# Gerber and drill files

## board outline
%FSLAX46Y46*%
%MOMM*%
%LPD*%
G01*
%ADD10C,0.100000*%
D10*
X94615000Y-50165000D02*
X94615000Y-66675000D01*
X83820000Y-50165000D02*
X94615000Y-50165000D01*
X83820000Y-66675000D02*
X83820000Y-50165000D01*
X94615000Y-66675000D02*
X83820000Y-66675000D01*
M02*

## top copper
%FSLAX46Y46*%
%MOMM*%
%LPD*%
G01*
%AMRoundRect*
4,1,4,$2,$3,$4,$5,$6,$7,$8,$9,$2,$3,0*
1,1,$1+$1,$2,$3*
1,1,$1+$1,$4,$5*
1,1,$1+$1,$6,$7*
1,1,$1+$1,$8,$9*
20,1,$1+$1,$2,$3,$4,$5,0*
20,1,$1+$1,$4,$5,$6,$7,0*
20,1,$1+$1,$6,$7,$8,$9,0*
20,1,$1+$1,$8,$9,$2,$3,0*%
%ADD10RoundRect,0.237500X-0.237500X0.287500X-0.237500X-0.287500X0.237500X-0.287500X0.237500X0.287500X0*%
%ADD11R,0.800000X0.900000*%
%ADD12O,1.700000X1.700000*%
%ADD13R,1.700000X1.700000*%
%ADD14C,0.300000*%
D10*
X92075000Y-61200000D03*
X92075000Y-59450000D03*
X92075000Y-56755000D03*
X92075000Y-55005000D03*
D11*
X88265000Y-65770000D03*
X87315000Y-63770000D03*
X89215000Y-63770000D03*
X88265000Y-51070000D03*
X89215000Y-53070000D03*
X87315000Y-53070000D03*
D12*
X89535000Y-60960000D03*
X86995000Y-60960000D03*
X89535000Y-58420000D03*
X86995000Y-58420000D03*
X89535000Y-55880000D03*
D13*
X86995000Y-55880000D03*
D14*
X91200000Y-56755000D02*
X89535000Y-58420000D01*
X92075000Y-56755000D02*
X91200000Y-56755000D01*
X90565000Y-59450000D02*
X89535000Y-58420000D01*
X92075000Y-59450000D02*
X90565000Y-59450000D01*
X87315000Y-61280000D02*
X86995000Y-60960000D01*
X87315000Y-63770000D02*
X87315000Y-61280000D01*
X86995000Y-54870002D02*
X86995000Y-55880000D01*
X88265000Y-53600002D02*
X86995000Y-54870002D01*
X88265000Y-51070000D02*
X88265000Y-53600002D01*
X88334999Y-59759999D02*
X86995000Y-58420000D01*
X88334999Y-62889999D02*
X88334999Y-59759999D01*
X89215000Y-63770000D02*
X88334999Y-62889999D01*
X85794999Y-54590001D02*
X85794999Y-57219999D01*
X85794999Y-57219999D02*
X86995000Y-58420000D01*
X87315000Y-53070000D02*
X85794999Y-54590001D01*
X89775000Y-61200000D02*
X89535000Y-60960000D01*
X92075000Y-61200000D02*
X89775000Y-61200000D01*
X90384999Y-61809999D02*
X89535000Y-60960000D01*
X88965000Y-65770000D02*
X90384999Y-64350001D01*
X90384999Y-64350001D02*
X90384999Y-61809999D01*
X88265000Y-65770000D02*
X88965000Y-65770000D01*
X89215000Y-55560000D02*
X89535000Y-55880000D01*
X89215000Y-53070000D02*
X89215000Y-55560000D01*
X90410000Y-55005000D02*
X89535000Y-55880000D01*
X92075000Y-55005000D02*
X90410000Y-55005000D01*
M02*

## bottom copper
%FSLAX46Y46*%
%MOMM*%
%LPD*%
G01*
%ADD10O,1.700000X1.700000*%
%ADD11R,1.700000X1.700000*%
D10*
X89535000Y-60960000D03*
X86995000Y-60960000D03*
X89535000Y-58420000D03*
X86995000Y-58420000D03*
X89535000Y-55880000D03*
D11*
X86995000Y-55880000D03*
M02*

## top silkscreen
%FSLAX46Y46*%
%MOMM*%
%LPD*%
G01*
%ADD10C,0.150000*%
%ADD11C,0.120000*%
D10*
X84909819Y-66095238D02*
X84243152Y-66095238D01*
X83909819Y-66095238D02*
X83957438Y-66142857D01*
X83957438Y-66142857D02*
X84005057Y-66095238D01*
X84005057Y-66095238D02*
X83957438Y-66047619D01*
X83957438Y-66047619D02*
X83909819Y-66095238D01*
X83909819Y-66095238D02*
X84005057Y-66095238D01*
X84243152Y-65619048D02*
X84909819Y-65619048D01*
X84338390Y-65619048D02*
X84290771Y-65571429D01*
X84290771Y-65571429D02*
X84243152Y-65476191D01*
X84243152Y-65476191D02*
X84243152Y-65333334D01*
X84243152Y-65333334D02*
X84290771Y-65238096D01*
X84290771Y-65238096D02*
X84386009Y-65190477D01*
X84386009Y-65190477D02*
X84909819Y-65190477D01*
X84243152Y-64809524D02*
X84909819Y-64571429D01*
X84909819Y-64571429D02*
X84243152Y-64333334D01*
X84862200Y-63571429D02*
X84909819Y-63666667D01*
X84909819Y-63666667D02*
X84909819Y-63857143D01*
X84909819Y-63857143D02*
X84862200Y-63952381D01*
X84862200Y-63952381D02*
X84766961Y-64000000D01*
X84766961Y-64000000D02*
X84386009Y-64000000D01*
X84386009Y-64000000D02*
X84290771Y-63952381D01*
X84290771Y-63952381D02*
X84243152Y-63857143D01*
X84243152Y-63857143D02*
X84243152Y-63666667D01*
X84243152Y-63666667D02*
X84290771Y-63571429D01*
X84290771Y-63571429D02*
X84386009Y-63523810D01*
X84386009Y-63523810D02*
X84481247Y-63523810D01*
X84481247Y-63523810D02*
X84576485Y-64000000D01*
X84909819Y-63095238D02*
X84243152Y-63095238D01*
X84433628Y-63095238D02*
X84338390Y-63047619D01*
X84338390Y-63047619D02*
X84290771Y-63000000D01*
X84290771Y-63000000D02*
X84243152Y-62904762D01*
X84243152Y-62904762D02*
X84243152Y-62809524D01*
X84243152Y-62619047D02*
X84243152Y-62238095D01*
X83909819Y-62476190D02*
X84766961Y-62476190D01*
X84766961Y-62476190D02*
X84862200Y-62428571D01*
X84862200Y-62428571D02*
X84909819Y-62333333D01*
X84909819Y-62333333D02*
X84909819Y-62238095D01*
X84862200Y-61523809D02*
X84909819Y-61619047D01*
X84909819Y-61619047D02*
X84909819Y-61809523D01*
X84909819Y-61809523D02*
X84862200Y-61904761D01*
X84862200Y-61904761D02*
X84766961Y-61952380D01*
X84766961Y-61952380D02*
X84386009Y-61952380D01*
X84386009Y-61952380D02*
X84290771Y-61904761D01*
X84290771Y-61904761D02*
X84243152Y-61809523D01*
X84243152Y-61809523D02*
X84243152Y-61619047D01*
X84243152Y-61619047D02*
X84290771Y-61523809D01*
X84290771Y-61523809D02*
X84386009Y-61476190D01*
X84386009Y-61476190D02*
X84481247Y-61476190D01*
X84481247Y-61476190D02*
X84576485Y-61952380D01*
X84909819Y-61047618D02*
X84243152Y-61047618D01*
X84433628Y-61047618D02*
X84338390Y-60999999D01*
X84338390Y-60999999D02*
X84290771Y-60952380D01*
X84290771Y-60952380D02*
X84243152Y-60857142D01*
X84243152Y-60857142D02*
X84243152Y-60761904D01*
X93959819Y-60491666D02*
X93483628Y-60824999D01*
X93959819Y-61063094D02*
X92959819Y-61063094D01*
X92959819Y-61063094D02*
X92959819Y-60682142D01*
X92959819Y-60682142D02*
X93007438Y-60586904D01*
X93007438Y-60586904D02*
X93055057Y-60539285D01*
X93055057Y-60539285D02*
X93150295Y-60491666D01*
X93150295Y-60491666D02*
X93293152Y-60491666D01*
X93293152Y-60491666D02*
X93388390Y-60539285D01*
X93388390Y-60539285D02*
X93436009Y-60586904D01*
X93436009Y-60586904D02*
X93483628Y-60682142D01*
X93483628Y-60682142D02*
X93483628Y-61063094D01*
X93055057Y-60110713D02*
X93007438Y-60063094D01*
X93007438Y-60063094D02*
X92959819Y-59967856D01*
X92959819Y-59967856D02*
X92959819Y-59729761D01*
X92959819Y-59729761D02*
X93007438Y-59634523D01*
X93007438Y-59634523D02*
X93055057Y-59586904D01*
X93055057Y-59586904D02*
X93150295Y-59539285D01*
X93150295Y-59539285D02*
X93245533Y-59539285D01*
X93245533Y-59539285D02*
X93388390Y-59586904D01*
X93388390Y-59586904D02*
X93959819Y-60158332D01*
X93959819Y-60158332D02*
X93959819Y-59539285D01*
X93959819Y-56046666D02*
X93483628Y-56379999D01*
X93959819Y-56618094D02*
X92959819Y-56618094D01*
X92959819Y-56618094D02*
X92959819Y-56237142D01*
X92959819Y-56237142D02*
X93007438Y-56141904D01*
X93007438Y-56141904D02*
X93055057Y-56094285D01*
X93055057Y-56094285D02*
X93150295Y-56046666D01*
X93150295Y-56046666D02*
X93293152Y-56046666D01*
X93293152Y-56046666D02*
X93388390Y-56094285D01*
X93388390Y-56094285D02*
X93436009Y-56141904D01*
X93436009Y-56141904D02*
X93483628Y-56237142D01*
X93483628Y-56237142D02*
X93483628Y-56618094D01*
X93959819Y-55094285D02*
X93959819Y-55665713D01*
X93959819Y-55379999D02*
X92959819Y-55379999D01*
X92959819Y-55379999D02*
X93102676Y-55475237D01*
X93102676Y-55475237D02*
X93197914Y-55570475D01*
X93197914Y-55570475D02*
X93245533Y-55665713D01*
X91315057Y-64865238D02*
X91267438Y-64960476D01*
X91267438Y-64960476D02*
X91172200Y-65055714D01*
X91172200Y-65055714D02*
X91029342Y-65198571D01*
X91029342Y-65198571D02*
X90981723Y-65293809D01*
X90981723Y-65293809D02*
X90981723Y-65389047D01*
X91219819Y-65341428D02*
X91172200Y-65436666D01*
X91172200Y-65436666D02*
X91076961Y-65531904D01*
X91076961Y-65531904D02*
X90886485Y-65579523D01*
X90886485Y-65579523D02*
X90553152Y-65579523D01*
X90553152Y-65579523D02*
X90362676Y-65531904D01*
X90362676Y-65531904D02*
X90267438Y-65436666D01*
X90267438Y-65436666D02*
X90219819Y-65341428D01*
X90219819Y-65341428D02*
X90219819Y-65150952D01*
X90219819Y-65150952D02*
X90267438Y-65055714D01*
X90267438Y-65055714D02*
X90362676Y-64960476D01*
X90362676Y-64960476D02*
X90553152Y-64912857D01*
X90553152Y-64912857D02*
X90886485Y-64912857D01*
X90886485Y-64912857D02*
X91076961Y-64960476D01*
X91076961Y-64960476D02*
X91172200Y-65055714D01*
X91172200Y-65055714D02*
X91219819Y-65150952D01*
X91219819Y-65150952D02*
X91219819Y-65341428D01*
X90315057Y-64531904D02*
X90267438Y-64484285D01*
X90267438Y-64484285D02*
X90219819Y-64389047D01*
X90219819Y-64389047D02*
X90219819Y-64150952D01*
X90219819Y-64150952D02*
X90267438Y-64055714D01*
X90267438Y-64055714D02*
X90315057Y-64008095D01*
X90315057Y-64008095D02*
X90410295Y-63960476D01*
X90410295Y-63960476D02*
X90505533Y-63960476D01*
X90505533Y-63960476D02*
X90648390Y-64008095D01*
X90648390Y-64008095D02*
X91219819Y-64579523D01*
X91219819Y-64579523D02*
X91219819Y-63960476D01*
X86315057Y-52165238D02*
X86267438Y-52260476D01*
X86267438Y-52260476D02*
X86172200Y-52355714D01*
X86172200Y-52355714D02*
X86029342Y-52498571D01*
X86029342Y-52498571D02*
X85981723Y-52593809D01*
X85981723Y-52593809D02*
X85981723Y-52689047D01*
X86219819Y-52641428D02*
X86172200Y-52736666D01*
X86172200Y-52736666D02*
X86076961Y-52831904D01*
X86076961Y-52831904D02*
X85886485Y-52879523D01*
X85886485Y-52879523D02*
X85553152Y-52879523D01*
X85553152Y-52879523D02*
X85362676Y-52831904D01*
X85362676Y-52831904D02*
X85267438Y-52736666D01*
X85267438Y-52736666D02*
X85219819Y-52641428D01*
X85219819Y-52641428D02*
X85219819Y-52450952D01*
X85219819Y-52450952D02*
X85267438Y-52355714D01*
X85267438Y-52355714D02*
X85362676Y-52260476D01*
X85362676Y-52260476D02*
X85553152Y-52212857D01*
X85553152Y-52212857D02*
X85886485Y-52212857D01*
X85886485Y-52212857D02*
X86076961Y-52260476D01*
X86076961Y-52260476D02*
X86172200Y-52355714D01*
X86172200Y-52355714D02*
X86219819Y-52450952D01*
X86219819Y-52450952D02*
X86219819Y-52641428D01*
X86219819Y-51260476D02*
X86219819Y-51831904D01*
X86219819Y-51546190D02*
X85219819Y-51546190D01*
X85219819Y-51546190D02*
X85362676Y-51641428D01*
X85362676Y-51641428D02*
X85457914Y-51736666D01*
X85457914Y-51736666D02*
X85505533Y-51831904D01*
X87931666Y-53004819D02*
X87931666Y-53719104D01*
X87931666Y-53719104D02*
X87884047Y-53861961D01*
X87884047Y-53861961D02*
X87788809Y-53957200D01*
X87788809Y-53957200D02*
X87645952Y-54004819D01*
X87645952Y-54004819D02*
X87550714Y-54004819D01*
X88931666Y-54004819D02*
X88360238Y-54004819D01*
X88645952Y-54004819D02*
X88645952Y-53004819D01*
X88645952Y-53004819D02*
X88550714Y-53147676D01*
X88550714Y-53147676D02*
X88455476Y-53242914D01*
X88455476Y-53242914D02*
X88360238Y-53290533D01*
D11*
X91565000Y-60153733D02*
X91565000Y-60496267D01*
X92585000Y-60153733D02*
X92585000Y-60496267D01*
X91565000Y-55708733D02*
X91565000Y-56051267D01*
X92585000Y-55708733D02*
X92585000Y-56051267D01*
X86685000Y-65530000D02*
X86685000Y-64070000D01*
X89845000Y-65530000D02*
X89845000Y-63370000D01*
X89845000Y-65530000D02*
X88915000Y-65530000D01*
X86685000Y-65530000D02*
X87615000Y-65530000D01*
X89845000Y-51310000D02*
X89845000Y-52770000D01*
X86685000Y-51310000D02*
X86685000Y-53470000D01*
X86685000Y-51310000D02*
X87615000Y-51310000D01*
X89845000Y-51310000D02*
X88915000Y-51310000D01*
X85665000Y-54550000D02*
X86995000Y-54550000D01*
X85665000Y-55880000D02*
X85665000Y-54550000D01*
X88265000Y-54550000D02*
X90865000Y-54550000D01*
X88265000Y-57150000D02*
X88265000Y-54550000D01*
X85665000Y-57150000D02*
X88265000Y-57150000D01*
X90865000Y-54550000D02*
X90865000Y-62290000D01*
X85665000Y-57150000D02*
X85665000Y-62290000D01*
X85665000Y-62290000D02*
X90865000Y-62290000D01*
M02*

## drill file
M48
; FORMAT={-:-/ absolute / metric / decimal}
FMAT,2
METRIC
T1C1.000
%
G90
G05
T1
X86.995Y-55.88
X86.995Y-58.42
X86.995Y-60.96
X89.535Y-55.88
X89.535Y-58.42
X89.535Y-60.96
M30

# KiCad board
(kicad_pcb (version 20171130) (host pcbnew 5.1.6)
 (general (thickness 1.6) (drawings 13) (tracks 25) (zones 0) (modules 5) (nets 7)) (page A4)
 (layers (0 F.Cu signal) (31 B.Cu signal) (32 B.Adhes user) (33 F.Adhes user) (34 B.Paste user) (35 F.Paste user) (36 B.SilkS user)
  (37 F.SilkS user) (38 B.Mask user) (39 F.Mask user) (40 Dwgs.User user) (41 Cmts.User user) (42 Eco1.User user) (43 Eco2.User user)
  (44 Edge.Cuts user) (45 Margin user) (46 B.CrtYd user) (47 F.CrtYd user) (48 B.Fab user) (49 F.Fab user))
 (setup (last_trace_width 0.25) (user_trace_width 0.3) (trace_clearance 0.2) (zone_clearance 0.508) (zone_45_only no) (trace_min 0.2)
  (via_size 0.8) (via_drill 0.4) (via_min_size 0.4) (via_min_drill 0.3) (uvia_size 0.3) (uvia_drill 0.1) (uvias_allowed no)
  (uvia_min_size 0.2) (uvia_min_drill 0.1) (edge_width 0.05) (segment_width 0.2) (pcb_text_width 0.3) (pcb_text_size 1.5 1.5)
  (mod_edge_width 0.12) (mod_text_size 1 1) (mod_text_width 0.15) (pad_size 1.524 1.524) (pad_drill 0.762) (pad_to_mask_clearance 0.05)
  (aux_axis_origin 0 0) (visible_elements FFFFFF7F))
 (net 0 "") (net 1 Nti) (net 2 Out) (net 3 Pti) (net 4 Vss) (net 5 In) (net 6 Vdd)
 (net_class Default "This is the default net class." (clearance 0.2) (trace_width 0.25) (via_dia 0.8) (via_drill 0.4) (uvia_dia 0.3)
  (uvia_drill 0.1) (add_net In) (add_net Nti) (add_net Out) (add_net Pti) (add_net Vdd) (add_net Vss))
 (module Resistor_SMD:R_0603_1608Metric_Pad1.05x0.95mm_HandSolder (layer F.Cu) (at 92.075 60.325 270)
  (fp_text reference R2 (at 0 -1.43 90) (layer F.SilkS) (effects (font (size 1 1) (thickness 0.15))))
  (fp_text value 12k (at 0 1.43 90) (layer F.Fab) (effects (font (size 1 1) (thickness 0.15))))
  (fp_line (start -0.171267 0.51) (end 0.171267 0.51) (layer F.SilkS) (width 0.12))
  (fp_line (start -0.171267 -0.51) (end 0.171267 -0.51) (layer F.SilkS) (width 0.12))
  (pad 2 smd roundrect (at 0.875 0 270) (size 1.05 0.95) (layers F.Cu F.Paste F.Mask) (roundrect_rratio 0.25) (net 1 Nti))
  (pad 1 smd roundrect (at -0.875 0 270) (size 1.05 0.95) (layers F.Cu F.Paste F.Mask) (roundrect_rratio 0.25) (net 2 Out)))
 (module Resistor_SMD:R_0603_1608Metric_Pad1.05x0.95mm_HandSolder (layer F.Cu) (at 92.075 55.88 270)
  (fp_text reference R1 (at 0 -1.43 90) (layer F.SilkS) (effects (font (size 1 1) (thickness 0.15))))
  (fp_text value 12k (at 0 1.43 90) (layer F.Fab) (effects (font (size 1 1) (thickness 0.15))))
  (fp_line (start -0.171267 0.51) (end 0.171267 0.51) (layer F.SilkS) (width 0.12))
  (fp_line (start -0.171267 -0.51) (end 0.171267 -0.51) (layer F.SilkS) (width 0.12))
  (pad 2 smd roundrect (at 0.875 0 270) (size 1.05 0.95) (layers F.Cu F.Paste F.Mask) (roundrect_rratio 0.25) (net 2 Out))
  (pad 1 smd roundrect (at -0.875 0 270) (size 1.05 0.95) (layers F.Cu F.Paste F.Mask) (roundrect_rratio 0.25) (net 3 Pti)))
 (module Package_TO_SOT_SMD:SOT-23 (layer F.Cu) (at 88.265 64.77 270)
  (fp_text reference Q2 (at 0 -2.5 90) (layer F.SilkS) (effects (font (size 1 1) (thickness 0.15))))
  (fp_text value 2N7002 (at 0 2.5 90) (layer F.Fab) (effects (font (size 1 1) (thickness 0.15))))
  (fp_line (start 0.76 1.58) (end -0.7 1.58) (layer F.SilkS) (width 0.12))
  (fp_line (start 0.76 -1.58) (end -1.4 -1.58) (layer F.SilkS) (width 0.12))
  (fp_line (start 0.76 -1.58) (end 0.76 -0.65) (layer F.SilkS) (width 0.12))
  (fp_line (start 0.76 1.58) (end 0.76 0.65) (layer F.SilkS) (width 0.12))
  (pad 3 smd rect (at 1 0 270) (size 0.9 0.8) (layers F.Cu F.Paste F.Mask) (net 1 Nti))
  (pad 2 smd rect (at -1 0.95 270) (size 0.9 0.8) (layers F.Cu F.Paste F.Mask) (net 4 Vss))
  (pad 1 smd rect (at -1 -0.95 270) (size 0.9 0.8) (layers F.Cu F.Paste F.Mask) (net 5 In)))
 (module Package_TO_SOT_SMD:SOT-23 (layer F.Cu) (at 88.265 52.07 90)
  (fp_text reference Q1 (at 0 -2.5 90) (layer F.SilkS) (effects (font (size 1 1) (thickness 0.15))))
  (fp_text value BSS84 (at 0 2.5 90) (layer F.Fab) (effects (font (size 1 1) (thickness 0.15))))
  (fp_line (start 0.76 1.58) (end -0.7 1.58) (layer F.SilkS) (width 0.12))
  (fp_line (start 0.76 -1.58) (end -1.4 -1.58) (layer F.SilkS) (width 0.12))
  (fp_line (start 0.76 -1.58) (end 0.76 -0.65) (layer F.SilkS) (width 0.12))
  (fp_line (start 0.76 1.58) (end 0.76 0.65) (layer F.SilkS) (width 0.12))
  (pad 3 smd rect (at 1 0 90) (size 0.9 0.8) (layers F.Cu F.Paste F.Mask) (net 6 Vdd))
  (pad 2 smd rect (at -1 0.95 90) (size 0.9 0.8) (layers F.Cu F.Paste F.Mask) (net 3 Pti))
  (pad 1 smd rect (at -1 -0.95 90) (size 0.9 0.8) (layers F.Cu F.Paste F.Mask) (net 5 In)))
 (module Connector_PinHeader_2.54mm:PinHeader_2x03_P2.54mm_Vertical (layer F.Cu) (at 86.995 55.88)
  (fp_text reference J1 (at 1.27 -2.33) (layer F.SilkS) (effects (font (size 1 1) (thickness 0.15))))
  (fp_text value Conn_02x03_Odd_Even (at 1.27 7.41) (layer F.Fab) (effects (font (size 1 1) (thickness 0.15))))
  (fp_line (start -1.33 -1.33) (end 0 -1.33) (layer F.SilkS) (width 0.12))
  (fp_line (start -1.33 0) (end -1.33 -1.33) (layer F.SilkS) (width 0.12))
  (fp_line (start 1.27 -1.33) (end 3.87 -1.33) (layer F.SilkS) (width 0.12))
  (fp_line (start 1.27 1.27) (end 1.27 -1.33) (layer F.SilkS) (width 0.12))
  (fp_line (start -1.33 1.27) (end 1.27 1.27) (layer F.SilkS) (width 0.12))
  (fp_line (start 3.87 -1.33) (end 3.87 6.41) (layer F.SilkS) (width 0.12))
  (fp_line (start -1.33 1.27) (end -1.33 6.41) (layer F.SilkS) (width 0.12))
  (fp_line (start -1.33 6.41) (end 3.87 6.41) (layer F.SilkS) (width 0.12))
  (pad 6 thru_hole oval (at 2.54 5.08) (size 1.7 1.7) (drill 1) (layers *.Cu *.Mask) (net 1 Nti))
  (pad 5 thru_hole oval (at 0 5.08) (size 1.7 1.7) (drill 1) (layers *.Cu *.Mask) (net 4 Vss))
  (pad 4 thru_hole oval (at 2.54 2.54) (size 1.7 1.7) (drill 1) (layers *.Cu *.Mask) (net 2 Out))
  (pad 3 thru_hole oval (at 0 2.54) (size 1.7 1.7) (drill 1) (layers *.Cu *.Mask) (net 5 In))
  (pad 2 thru_hole oval (at 2.54 0) (size 1.7 1.7) (drill 1) (layers *.Cu *.Mask) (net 3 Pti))
  (pad 1 thru_hole rect (at 0 0) (size 1.7 1.7) (drill 1) (layers *.Cu *.Mask) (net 6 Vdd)))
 (gr_line (start 94.615 50.165) (end 94.615 66.675) (layer Edge.Cuts) (width 0.1))
 (gr_line (start 83.82 50.165) (end 94.615 50.165) (layer Edge.Cuts) (width 0.1))
 (gr_line (start 83.82 66.675) (end 83.82 50.165) (layer Edge.Cuts) (width 0.1))
 (gr_line (start 94.615 66.675) (end 83.82 66.675) (layer Edge.Cuts) (width 0.1))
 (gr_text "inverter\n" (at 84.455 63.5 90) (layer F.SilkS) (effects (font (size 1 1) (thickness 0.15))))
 (segment (start 91.2 56.755) (end 89.535 58.42) (width 0.3) (layer F.Cu) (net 2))
 (segment (start 92.075 56.755) (end 91.2 56.755) (width 0.3) (layer F.Cu) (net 2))
 (segment (start 90.565 59.45) (end 89.535 58.42) (width 0.3) (layer F.Cu) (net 2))
 (segment (start 92.075 59.45) (end 90.565 59.45) (width 0.3) (layer F.Cu) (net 2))
 (segment (start 87.315 61.28) (end 86.995 60.96) (width 0.3) (layer F.Cu) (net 4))
 (segment (start 87.315 63.77) (end 87.315 61.28) (width 0.3) (layer F.Cu) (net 4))
 (segment (start 86.995 54.870002) (end 86.995 55.88) (width 0.3) (layer F.Cu) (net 6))
 (segment (start 88.265 53.600002) (end 86.995 54.870002) (width 0.3) (layer F.Cu) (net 6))
 (segment (start 88.265 51.07) (end 88.265 53.600002) (width 0.3) (layer F.Cu) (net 6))
 (segment (start 88.334999 59.759999) (end 86.995 58.42) (width 0.3) (layer F.Cu) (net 5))
 (segment (start 88.334999 62.889999) (end 88.334999 59.759999) (width 0.3) (layer F.Cu) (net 5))
 (segment (start 89.215 63.77) (end 88.334999 62.889999) (width 0.3) (layer F.Cu) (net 5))
 (segment (start 85.794999 54.590001) (end 85.794999 57.219999) (width 0.3) (layer F.Cu) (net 5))
 (segment (start 85.794999 57.219999) (end 86.995 58.42) (width 0.3) (layer F.Cu) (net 5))
 (segment (start 87.315 53.07) (end 85.794999 54.590001) (width 0.3) (layer F.Cu) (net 5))
 (segment (start 89.775 61.2) (end 89.535 60.96) (width 0.3) (layer F.Cu) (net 1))
 (segment (start 92.075 61.2) (end 89.775 61.2) (width 0.3) (layer F.Cu) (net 1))
 (segment (start 90.384999 61.809999) (end 89.535 60.96) (width 0.3) (layer F.Cu) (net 1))
 (segment (start 88.965 65.77) (end 90.384999 64.350001) (width 0.3) (layer F.Cu) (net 1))
 (segment (start 90.384999 64.350001) (end 90.384999 61.809999) (width 0.3) (layer F.Cu) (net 1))
 (segment (start 88.265 65.77) (end 88.965 65.77) (width 0.3) (layer F.Cu) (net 1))
 (segment (start 89.215 55.56) (end 89.535 55.88) (width 0.3) (layer F.Cu) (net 3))
 (segment (start 89.215 53.07) (end 89.215 55.56) (width 0.3) (layer F.Cu) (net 3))
 (segment (start 90.41 55.005) (end 89.535 55.88) (width 0.3) (layer F.Cu) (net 3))
 (segment (start 92.075 55.005) (end 90.41 55.005) (width 0.3) (layer F.Cu) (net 3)))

